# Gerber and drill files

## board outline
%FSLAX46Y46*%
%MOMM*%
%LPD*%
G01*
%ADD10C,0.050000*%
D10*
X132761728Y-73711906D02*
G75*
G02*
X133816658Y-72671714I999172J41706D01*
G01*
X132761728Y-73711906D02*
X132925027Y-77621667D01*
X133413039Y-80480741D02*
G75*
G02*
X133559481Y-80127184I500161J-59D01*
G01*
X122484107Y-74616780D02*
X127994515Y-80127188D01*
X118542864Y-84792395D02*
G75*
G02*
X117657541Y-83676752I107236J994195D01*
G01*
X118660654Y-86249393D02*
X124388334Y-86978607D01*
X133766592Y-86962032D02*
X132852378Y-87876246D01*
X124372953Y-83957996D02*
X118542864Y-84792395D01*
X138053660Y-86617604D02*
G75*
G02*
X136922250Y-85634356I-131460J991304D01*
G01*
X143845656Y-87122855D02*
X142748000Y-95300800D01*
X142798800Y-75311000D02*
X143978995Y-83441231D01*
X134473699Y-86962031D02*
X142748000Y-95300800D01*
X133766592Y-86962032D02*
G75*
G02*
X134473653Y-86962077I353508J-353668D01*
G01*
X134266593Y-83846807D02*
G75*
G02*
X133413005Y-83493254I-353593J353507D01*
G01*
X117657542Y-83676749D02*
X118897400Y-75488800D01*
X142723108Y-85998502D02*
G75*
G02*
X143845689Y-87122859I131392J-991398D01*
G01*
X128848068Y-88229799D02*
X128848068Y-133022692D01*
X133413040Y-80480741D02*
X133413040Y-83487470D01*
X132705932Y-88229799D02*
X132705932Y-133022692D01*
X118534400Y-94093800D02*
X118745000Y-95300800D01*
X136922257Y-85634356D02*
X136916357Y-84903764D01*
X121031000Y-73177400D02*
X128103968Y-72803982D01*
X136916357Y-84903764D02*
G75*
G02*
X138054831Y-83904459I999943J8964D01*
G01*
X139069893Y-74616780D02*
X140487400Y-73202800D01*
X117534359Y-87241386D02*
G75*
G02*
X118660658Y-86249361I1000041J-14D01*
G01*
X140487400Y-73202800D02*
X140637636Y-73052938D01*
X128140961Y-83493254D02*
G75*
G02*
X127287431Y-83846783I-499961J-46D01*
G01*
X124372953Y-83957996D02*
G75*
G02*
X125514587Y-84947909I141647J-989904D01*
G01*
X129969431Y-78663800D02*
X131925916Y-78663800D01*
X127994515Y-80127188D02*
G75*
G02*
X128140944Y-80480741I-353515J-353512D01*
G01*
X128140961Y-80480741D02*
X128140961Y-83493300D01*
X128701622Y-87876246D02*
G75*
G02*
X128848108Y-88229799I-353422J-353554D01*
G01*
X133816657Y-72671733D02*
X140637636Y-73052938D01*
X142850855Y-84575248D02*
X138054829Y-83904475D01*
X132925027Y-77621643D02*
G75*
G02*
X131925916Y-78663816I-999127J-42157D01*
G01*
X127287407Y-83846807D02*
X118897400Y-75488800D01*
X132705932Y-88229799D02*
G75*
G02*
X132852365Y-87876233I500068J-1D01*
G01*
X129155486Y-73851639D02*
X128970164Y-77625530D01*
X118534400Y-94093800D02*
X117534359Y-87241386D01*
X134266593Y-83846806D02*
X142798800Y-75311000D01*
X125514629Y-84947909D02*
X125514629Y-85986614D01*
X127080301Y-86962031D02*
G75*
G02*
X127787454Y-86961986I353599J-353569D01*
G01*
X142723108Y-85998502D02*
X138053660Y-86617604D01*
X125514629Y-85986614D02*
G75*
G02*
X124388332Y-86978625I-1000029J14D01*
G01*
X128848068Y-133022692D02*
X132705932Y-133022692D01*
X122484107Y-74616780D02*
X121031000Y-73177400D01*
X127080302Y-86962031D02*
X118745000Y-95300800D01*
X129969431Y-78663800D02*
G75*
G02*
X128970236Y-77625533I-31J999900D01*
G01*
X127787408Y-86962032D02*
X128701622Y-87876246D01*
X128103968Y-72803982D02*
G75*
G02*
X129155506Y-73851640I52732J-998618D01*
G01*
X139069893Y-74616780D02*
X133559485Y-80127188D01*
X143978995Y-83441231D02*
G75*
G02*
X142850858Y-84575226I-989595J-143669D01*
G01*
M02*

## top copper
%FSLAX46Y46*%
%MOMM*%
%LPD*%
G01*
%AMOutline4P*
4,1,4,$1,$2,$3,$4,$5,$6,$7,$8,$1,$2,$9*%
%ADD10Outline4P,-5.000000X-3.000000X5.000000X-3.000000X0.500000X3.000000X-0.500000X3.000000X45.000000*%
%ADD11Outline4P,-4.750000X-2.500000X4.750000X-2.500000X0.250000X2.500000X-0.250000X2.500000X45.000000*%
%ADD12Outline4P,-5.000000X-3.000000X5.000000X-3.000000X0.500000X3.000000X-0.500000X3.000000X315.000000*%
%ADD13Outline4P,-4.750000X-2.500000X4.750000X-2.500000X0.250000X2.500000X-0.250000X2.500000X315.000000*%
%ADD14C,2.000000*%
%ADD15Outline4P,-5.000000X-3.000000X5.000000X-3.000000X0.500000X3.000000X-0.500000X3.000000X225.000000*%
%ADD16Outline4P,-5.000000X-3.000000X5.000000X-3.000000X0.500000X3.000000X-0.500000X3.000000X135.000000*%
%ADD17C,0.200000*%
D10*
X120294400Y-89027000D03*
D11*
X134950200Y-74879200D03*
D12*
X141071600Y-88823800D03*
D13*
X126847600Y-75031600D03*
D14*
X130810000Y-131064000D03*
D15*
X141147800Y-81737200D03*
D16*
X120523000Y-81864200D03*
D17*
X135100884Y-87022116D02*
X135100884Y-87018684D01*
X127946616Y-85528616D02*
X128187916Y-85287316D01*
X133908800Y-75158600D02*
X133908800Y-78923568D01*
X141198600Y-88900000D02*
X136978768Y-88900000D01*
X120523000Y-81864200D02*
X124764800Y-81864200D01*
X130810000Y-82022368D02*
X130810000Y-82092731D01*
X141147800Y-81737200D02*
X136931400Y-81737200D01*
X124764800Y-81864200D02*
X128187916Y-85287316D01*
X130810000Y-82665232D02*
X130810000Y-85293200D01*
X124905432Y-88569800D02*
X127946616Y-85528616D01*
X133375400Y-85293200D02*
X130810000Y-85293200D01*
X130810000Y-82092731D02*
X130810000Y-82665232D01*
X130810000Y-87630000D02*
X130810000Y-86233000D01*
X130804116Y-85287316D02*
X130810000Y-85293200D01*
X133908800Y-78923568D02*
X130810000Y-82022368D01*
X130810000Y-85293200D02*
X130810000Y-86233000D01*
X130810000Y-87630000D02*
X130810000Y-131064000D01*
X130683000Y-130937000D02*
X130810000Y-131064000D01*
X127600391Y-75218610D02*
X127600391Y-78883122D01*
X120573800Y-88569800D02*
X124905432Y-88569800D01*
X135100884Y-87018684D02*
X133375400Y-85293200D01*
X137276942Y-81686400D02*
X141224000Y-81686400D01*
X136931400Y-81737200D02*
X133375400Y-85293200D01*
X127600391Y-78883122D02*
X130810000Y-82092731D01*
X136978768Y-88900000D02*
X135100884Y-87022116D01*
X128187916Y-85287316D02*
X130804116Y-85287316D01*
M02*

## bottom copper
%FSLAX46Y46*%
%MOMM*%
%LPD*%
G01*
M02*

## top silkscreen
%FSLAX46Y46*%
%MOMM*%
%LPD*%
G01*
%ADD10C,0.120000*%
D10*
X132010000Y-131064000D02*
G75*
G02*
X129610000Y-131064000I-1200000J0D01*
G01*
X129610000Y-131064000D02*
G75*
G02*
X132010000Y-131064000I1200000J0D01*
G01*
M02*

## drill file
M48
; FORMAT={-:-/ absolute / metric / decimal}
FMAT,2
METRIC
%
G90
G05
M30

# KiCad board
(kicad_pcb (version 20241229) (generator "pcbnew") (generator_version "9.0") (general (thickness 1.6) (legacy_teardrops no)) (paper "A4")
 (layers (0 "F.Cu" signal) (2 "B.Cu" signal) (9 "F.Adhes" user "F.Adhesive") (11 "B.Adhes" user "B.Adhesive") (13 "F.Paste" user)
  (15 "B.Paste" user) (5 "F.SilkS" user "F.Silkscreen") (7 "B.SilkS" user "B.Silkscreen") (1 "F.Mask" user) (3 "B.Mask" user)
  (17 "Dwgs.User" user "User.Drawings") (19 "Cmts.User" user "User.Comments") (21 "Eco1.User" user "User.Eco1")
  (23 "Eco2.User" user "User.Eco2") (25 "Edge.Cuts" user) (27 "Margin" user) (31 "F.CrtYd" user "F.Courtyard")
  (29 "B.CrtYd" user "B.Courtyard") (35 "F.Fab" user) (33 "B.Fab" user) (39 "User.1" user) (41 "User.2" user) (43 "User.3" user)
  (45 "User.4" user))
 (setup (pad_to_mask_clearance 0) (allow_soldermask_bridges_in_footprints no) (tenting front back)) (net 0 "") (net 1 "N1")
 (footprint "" (layer "F.Cu") (at 120.2944 89.027 -90)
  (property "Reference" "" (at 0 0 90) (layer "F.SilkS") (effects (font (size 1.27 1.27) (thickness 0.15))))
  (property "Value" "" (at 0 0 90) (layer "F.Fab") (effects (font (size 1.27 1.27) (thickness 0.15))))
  (pad "1" smd trapezoid (at 0 0 45) (size 5.5 6) (rect_delta 0 4.5) (layers "F.Cu" "F.Mask") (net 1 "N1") (clearance 0.1)))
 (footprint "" (layer "F.Cu") (at 134.9502 74.8792)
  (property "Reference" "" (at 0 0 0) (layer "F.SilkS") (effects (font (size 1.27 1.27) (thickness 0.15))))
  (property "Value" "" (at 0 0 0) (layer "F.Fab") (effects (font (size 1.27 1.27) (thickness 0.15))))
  (pad "1" smd trapezoid (at 0 0 45) (size 5 5) (rect_delta 0 4.5) (layers "F.Cu" "F.Mask") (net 1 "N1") (clearance 0.1)))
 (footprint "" (layer "F.Cu") (at 141.0716 88.8238)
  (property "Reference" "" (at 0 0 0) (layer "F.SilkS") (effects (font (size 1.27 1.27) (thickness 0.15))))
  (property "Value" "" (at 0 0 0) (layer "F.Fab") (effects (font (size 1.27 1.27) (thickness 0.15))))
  (pad "1" smd trapezoid (at 0 0 315) (size 5.5 6) (rect_delta 0 4.5) (layers "F.Cu" "F.Mask") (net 1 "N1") (clearance 0.1)))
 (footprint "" (layer "F.Cu") (at 126.8476 75.0316 180)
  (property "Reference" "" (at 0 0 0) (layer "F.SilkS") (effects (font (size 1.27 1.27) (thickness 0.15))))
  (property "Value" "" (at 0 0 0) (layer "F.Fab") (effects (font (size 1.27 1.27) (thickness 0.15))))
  (pad "1" smd trapezoid (at 0 0 315) (size 5 5) (rect_delta 0 4.5) (layers "F.Cu" "F.Mask") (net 1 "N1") (clearance 0.1)))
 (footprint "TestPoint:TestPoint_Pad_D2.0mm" (layer "F.Cu") (at 130.81 131.064)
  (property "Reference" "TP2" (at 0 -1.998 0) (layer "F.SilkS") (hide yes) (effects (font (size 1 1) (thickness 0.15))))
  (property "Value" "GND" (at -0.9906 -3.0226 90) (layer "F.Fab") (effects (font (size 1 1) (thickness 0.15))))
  (fp_circle (center 0 0) (end 0 1.2) (stroke (width 0.12) (type solid)) (fill no) (layer "F.SilkS"))
  (pad "1" smd circle (at 0 0) (size 2 2) (layers "F.Cu" "F.Mask") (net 1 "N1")))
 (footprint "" (layer "F.Cu") (at 141.1478 81.7372)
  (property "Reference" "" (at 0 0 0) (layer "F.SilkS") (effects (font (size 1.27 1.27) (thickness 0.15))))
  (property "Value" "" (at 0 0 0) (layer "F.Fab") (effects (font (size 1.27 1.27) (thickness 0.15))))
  (pad "1" smd trapezoid (at 0 0 225) (size 5.5 6) (rect_delta 0 4.5) (layers "F.Cu" "F.Mask") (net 1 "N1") (clearance 0.1)))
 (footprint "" (layer "F.Cu") (at 120.523 81.8642)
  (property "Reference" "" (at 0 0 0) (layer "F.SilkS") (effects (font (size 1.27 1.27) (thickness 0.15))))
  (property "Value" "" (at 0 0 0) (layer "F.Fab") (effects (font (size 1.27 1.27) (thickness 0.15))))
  (pad "1" smd trapezoid (at 0 0 135) (size 5.5 6) (rect_delta 0 4.5) (layers "F.Cu" "F.Mask") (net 1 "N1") (clearance 0.1)))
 (gr_arc (start 132.761728 73.711906) (mid 133.058755 72.958107) (end 133.816657 72.671733) (stroke (width 0.05) (type default))
  (layer "Edge.Cuts"))
 (gr_line (start 132.761728 73.711906) (end 132.925027 77.621667) (stroke (width 0.05) (type default)) (layer "Edge.Cuts"))
 (gr_arc (start 133.413039 80.480741) (mid 133.451112 80.289409) (end 133.559485 80.127188) (stroke (width 0.05) (type default))
  (layer "Edge.Cuts"))
 (gr_line (start 122.484107 74.61678) (end 127.994515 80.127188) (stroke (width 0.05) (type solid)) (layer "Edge.Cuts"))
 (gr_arc (start 118.542864 84.792395) (mid 117.866801 84.419784) (end 117.657517 83.676749) (stroke (width 0.05) (type default))
  (layer "Edge.Cuts"))
 (gr_line (start 118.660654 86.249393) (end 124.388334 86.978607) (stroke (width 0.05) (type solid)) (layer "Edge.Cuts"))
 (gr_line (start 133.766592 86.962032) (end 132.852378 87.876246) (stroke (width 0.05) (type solid)) (layer "Edge.Cuts"))
 (gr_line (start 124.372953 83.957996) (end 118.542864 84.792395) (stroke (width 0.05) (type default)) (layer "Edge.Cuts"))
 (gr_arc (start 138.05366 86.617604) (mid 137.266256 86.381086) (end 136.922257 85.634356) (stroke (width 0.05) (type default))
  (layer "Edge.Cuts"))
 (gr_line (start 143.845656 87.122855) (end 142.748 95.3008) (stroke (width 0.05) (type default)) (layer "Edge.Cuts"))
 (gr_line (start 142.7988 75.311) (end 143.978995 83.441231) (stroke (width 0.05) (type default)) (layer "Edge.Cuts"))
 (gr_line (start 134.473699 86.962031) (end 142.748 95.3008) (stroke (width 0.05) (type default)) (layer "Edge.Cuts"))
 (gr_arc (start 133.766592 86.962032) (mid 134.120132 86.815622) (end 134.473699 86.962031) (stroke (width 0.05) (type default))
  (layer "Edge.Cuts"))
 (gr_arc (start 134.266593 83.846807) (mid 133.721667 83.955238) (end 133.413039 83.493254) (stroke (width 0.05) (type default))
  (layer "Edge.Cuts"))
 (gr_line (start 117.657542 83.676749) (end 118.8974 75.4888) (stroke (width 0.05) (type default)) (layer "Edge.Cuts"))
 (gr_arc (start 142.723108 85.998502) (mid 143.562173 86.283306) (end 143.845656 87.122855) (stroke (width 0.05) (type default))
  (layer "Edge.Cuts"))
 (gr_line (start 128.848068 88.229799) (end 128.848068 133.022692) (stroke (width 0.05) (type solid)) (layer "Edge.Cuts"))
 (gr_line (start 133.41304 80.480741) (end 133.41304 83.48747) (stroke (width 0.05) (type default)) (layer "Edge.Cuts"))
 (gr_line (start 132.705932 88.229799) (end 132.705932 133.022692) (stroke (width 0.05) (type solid)) (layer "Edge.Cuts"))
 (gr_line (start 118.5344 94.0938) (end 118.745 95.3008) (stroke (width 0.05) (type default)) (layer "Edge.Cuts"))
 (gr_line (start 136.922257 85.634356) (end 136.916357 84.903764) (stroke (width 0.05) (type default)) (layer "Edge.Cuts"))
 (gr_line (start 121.031 73.1774) (end 128.103968 72.803982) (stroke (width 0.05) (type default)) (layer "Edge.Cuts"))
 (gr_arc (start 136.916357 84.903764) (mid 137.256633 84.143264) (end 138.054829 83.904475) (stroke (width 0.05) (type default))
  (layer "Edge.Cuts"))
 (gr_line (start 139.069893 74.61678) (end 140.4874 73.2028) (stroke (width 0.05) (type default)) (layer "Edge.Cuts"))
 (gr_arc (start 117.534359 87.241386) (mid 117.873414 86.490947) (end 118.660654 86.249393) (stroke (width 0.05) (type default))
  (layer "Edge.Cuts"))
 (gr_line (start 140.4874 73.2028) (end 140.637636 73.052938) (stroke (width 0.05) (type default)) (layer "Edge.Cuts"))
 (gr_arc (start 128.140961 83.493254) (mid 127.832302 83.955194) (end 127.287407 83.846807) (stroke (width 0.05) (type default))
  (layer "Edge.Cuts"))
 (gr_arc (start 124.372953 83.957996) (mid 125.169734 84.192371) (end 125.514629 84.947909) (stroke (width 0.05) (type default))
  (layer "Edge.Cuts"))
 (gr_line (start 129.969431 78.6638) (end 131.925916 78.6638) (stroke (width 0.05) (type default)) (layer "Edge.Cuts"))
 (gr_arc (start 127.994515 80.127188) (mid 128.102901 80.2894) (end 128.140961 80.480741) (stroke (width 0.05) (type default))
  (layer "Edge.Cuts"))
 (gr_line (start 128.140961 80.480741) (end 128.140961 83.4933) (stroke (width 0.05) (type default)) (layer "Edge.Cuts"))
 (gr_arc (start 128.701622 87.876246) (mid 128.810015 88.038456) (end 128.848068 88.229799) (stroke (width 0.05) (type default))
  (layer "Edge.Cuts"))
 (gr_line (start 133.816657 72.671733) (end 140.637636 73.052938) (stroke (width 0.05) (type default)) (layer "Edge.Cuts"))
 (gr_line (start 142.850855 84.575248) (end 138.054829 83.904475) (stroke (width 0.05) (type default)) (layer "Edge.Cuts"))
 (gr_arc (start 132.925027 77.621643) (mid 132.647774 78.355842) (end 131.925916 78.6638) (stroke (width 0.05) (type default))
  (layer "Edge.Cuts"))
 (gr_line (start 127.287407 83.846807) (end 118.8974 75.4888) (stroke (width 0.05) (type default)) (layer "Edge.Cuts"))
 (gr_arc (start 132.705932 88.229799) (mid 132.743994 88.03846) (end 132.852378 87.876246) (stroke (width 0.05) (type default))
  (layer "Edge.Cuts"))
 (gr_line (start 129.155486 73.851639) (end 128.970164 77.62553) (stroke (width 0.05) (type default)) (layer "Edge.Cuts"))
 (gr_line (start 118.5344 94.0938) (end 117.534359 87.241386) (stroke (width 0.05) (type default)) (layer "Edge.Cuts"))
 (gr_line (start 134.266593 83.846806) (end 142.7988 75.311) (stroke (width 0.05) (type default)) (layer "Edge.Cuts"))
 (gr_line (start 125.514629 84.947909) (end 125.514629 85.986614) (stroke (width 0.05) (type default)) (layer "Edge.Cuts"))
 (gr_arc (start 127.080301 86.962031) (mid 127.433855 86.815585) (end 127.787408 86.962032) (stroke (width 0.05) (type default))
  (layer "Edge.Cuts"))
 (gr_line (start 142.723108 85.998502) (end 138.05366 86.617604) (stroke (width 0.05) (type default)) (layer "Edge.Cuts"))
 (gr_arc (start 125.514629 85.986614) (mid 125.175574 86.737048) (end 124.388334 86.978607) (stroke (width 0.05) (type default))
  (layer "Edge.Cuts"))
 (gr_line (start 128.848068 133.022692) (end 132.705932 133.022692) (stroke (width 0.05) (type default)) (layer "Edge.Cuts"))
 (gr_line (start 122.484107 74.61678) (end 121.031 73.1774) (stroke (width 0.05) (type default)) (layer "Edge.Cuts"))
 (gr_line (start 127.080302 86.962031) (end 118.745 95.3008) (stroke (width 0.05) (type default)) (layer "Edge.Cuts"))
 (gr_arc (start 129.969431 78.6638) (mid 129.2489 78.357255) (end 128.970164 77.62553) (stroke (width 0.05) (type default))
  (layer "Edge.Cuts"))
 (gr_line (start 127.787408 86.962032) (end 128.701622 87.876246) (stroke (width 0.05) (type solid)) (layer "Edge.Cuts"))
 (gr_arc (start 128.103968 72.803982) (mid 128.862495 73.094185) (end 129.155486 73.851639) (stroke (width 0.05) (type default))
  (layer "Edge.Cuts"))
 (gr_line (start 139.069893 74.61678) (end 133.559485 80.127188) (stroke (width 0.05) (type solid)) (layer "Edge.Cuts"))
 (gr_arc (start 143.978995 83.441231) (mid 143.698309 84.290155) (end 142.850855 84.575248) (stroke (width 0.05) (type default))
  (layer "Edge.Cuts"))
 (segment (start 135.100884 87.022116) (end 135.100884 87.018684) (width 0.2) (layer "F.Cu") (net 1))
 (segment (start 127.946616 85.528616) (end 128.187916 85.287316) (width 0.2) (layer "F.Cu") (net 1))
 (segment (start 133.9088 75.1586) (end 133.9088 78.923568) (width 0.2) (layer "F.Cu") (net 1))
 (segment (start 141.1986 88.9) (end 136.978768 88.9) (width 0.2) (layer "F.Cu") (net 1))
 (segment (start 120.523 81.8642) (end 124.7648 81.8642) (width 0.2) (layer "F.Cu") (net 1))
 (segment (start 130.81 82.022368) (end 130.81 82.092731) (width 0.2) (layer "F.Cu") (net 1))
 (segment (start 141.1478 81.7372) (end 136.9314 81.7372) (width 0.2) (layer "F.Cu") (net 1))
 (segment (start 124.7648 81.8642) (end 128.187916 85.287316) (width 0.2) (layer "F.Cu") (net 1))
 (segment (start 130.81 82.665232) (end 130.81 85.2932) (width 0.2) (layer "F.Cu") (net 1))
 (segment (start 124.905432 88.5698) (end 127.946616 85.528616) (width 0.2) (layer "F.Cu") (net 1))
 (segment (start 133.3754 85.2932) (end 130.81 85.2932) (width 0.2) (layer "F.Cu") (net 1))
 (segment (start 130.81 82.092731) (end 130.81 82.665232) (width 0.2) (layer "F.Cu") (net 1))
 (segment (start 130.81 87.63) (end 130.81 86.233) (width 0.2) (layer "F.Cu") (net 1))
 (segment (start 130.804116 85.287316) (end 130.81 85.2932) (width 0.2) (layer "F.Cu") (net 1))
 (segment (start 133.9088 78.923568) (end 130.81 82.022368) (width 0.2) (layer "F.Cu") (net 1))
 (segment (start 130.81 85.2932) (end 130.81 86.233) (width 0.2) (layer "F.Cu") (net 1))
 (segment (start 130.81 87.63) (end 130.81 131.064) (width 0.2) (layer "F.Cu") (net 1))
 (segment (start 130.683 130.937) (end 130.81 131.064) (width 0.2) (layer "F.Cu") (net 1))
 (segment (start 127.600391 75.21861) (end 127.600391 78.883122) (width 0.2) (layer "F.Cu") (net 1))
 (segment (start 120.5738 88.5698) (end 124.905432 88.5698) (width 0.2) (layer "F.Cu") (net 1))
 (segment (start 135.100884 87.018684) (end 133.3754 85.2932) (width 0.2) (layer "F.Cu") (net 1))
 (segment (start 137.276942 81.6864) (end 141.224 81.6864) (width 0.2) (layer "F.Cu") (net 1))
 (segment (start 136.9314 81.7372) (end 133.3754 85.2932) (width 0.2) (layer "F.Cu") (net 1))
 (segment (start 127.600391 78.883122) (end 130.81 82.092731) (width 0.2) (layer "F.Cu") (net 1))
 (segment (start 136.978768 88.9) (end 135.100884 87.022116) (width 0.2) (layer "F.Cu") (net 1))
 (segment (start 128.187916 85.287316) (end 130.804116 85.287316) (width 0.2) (layer "F.Cu") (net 1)))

